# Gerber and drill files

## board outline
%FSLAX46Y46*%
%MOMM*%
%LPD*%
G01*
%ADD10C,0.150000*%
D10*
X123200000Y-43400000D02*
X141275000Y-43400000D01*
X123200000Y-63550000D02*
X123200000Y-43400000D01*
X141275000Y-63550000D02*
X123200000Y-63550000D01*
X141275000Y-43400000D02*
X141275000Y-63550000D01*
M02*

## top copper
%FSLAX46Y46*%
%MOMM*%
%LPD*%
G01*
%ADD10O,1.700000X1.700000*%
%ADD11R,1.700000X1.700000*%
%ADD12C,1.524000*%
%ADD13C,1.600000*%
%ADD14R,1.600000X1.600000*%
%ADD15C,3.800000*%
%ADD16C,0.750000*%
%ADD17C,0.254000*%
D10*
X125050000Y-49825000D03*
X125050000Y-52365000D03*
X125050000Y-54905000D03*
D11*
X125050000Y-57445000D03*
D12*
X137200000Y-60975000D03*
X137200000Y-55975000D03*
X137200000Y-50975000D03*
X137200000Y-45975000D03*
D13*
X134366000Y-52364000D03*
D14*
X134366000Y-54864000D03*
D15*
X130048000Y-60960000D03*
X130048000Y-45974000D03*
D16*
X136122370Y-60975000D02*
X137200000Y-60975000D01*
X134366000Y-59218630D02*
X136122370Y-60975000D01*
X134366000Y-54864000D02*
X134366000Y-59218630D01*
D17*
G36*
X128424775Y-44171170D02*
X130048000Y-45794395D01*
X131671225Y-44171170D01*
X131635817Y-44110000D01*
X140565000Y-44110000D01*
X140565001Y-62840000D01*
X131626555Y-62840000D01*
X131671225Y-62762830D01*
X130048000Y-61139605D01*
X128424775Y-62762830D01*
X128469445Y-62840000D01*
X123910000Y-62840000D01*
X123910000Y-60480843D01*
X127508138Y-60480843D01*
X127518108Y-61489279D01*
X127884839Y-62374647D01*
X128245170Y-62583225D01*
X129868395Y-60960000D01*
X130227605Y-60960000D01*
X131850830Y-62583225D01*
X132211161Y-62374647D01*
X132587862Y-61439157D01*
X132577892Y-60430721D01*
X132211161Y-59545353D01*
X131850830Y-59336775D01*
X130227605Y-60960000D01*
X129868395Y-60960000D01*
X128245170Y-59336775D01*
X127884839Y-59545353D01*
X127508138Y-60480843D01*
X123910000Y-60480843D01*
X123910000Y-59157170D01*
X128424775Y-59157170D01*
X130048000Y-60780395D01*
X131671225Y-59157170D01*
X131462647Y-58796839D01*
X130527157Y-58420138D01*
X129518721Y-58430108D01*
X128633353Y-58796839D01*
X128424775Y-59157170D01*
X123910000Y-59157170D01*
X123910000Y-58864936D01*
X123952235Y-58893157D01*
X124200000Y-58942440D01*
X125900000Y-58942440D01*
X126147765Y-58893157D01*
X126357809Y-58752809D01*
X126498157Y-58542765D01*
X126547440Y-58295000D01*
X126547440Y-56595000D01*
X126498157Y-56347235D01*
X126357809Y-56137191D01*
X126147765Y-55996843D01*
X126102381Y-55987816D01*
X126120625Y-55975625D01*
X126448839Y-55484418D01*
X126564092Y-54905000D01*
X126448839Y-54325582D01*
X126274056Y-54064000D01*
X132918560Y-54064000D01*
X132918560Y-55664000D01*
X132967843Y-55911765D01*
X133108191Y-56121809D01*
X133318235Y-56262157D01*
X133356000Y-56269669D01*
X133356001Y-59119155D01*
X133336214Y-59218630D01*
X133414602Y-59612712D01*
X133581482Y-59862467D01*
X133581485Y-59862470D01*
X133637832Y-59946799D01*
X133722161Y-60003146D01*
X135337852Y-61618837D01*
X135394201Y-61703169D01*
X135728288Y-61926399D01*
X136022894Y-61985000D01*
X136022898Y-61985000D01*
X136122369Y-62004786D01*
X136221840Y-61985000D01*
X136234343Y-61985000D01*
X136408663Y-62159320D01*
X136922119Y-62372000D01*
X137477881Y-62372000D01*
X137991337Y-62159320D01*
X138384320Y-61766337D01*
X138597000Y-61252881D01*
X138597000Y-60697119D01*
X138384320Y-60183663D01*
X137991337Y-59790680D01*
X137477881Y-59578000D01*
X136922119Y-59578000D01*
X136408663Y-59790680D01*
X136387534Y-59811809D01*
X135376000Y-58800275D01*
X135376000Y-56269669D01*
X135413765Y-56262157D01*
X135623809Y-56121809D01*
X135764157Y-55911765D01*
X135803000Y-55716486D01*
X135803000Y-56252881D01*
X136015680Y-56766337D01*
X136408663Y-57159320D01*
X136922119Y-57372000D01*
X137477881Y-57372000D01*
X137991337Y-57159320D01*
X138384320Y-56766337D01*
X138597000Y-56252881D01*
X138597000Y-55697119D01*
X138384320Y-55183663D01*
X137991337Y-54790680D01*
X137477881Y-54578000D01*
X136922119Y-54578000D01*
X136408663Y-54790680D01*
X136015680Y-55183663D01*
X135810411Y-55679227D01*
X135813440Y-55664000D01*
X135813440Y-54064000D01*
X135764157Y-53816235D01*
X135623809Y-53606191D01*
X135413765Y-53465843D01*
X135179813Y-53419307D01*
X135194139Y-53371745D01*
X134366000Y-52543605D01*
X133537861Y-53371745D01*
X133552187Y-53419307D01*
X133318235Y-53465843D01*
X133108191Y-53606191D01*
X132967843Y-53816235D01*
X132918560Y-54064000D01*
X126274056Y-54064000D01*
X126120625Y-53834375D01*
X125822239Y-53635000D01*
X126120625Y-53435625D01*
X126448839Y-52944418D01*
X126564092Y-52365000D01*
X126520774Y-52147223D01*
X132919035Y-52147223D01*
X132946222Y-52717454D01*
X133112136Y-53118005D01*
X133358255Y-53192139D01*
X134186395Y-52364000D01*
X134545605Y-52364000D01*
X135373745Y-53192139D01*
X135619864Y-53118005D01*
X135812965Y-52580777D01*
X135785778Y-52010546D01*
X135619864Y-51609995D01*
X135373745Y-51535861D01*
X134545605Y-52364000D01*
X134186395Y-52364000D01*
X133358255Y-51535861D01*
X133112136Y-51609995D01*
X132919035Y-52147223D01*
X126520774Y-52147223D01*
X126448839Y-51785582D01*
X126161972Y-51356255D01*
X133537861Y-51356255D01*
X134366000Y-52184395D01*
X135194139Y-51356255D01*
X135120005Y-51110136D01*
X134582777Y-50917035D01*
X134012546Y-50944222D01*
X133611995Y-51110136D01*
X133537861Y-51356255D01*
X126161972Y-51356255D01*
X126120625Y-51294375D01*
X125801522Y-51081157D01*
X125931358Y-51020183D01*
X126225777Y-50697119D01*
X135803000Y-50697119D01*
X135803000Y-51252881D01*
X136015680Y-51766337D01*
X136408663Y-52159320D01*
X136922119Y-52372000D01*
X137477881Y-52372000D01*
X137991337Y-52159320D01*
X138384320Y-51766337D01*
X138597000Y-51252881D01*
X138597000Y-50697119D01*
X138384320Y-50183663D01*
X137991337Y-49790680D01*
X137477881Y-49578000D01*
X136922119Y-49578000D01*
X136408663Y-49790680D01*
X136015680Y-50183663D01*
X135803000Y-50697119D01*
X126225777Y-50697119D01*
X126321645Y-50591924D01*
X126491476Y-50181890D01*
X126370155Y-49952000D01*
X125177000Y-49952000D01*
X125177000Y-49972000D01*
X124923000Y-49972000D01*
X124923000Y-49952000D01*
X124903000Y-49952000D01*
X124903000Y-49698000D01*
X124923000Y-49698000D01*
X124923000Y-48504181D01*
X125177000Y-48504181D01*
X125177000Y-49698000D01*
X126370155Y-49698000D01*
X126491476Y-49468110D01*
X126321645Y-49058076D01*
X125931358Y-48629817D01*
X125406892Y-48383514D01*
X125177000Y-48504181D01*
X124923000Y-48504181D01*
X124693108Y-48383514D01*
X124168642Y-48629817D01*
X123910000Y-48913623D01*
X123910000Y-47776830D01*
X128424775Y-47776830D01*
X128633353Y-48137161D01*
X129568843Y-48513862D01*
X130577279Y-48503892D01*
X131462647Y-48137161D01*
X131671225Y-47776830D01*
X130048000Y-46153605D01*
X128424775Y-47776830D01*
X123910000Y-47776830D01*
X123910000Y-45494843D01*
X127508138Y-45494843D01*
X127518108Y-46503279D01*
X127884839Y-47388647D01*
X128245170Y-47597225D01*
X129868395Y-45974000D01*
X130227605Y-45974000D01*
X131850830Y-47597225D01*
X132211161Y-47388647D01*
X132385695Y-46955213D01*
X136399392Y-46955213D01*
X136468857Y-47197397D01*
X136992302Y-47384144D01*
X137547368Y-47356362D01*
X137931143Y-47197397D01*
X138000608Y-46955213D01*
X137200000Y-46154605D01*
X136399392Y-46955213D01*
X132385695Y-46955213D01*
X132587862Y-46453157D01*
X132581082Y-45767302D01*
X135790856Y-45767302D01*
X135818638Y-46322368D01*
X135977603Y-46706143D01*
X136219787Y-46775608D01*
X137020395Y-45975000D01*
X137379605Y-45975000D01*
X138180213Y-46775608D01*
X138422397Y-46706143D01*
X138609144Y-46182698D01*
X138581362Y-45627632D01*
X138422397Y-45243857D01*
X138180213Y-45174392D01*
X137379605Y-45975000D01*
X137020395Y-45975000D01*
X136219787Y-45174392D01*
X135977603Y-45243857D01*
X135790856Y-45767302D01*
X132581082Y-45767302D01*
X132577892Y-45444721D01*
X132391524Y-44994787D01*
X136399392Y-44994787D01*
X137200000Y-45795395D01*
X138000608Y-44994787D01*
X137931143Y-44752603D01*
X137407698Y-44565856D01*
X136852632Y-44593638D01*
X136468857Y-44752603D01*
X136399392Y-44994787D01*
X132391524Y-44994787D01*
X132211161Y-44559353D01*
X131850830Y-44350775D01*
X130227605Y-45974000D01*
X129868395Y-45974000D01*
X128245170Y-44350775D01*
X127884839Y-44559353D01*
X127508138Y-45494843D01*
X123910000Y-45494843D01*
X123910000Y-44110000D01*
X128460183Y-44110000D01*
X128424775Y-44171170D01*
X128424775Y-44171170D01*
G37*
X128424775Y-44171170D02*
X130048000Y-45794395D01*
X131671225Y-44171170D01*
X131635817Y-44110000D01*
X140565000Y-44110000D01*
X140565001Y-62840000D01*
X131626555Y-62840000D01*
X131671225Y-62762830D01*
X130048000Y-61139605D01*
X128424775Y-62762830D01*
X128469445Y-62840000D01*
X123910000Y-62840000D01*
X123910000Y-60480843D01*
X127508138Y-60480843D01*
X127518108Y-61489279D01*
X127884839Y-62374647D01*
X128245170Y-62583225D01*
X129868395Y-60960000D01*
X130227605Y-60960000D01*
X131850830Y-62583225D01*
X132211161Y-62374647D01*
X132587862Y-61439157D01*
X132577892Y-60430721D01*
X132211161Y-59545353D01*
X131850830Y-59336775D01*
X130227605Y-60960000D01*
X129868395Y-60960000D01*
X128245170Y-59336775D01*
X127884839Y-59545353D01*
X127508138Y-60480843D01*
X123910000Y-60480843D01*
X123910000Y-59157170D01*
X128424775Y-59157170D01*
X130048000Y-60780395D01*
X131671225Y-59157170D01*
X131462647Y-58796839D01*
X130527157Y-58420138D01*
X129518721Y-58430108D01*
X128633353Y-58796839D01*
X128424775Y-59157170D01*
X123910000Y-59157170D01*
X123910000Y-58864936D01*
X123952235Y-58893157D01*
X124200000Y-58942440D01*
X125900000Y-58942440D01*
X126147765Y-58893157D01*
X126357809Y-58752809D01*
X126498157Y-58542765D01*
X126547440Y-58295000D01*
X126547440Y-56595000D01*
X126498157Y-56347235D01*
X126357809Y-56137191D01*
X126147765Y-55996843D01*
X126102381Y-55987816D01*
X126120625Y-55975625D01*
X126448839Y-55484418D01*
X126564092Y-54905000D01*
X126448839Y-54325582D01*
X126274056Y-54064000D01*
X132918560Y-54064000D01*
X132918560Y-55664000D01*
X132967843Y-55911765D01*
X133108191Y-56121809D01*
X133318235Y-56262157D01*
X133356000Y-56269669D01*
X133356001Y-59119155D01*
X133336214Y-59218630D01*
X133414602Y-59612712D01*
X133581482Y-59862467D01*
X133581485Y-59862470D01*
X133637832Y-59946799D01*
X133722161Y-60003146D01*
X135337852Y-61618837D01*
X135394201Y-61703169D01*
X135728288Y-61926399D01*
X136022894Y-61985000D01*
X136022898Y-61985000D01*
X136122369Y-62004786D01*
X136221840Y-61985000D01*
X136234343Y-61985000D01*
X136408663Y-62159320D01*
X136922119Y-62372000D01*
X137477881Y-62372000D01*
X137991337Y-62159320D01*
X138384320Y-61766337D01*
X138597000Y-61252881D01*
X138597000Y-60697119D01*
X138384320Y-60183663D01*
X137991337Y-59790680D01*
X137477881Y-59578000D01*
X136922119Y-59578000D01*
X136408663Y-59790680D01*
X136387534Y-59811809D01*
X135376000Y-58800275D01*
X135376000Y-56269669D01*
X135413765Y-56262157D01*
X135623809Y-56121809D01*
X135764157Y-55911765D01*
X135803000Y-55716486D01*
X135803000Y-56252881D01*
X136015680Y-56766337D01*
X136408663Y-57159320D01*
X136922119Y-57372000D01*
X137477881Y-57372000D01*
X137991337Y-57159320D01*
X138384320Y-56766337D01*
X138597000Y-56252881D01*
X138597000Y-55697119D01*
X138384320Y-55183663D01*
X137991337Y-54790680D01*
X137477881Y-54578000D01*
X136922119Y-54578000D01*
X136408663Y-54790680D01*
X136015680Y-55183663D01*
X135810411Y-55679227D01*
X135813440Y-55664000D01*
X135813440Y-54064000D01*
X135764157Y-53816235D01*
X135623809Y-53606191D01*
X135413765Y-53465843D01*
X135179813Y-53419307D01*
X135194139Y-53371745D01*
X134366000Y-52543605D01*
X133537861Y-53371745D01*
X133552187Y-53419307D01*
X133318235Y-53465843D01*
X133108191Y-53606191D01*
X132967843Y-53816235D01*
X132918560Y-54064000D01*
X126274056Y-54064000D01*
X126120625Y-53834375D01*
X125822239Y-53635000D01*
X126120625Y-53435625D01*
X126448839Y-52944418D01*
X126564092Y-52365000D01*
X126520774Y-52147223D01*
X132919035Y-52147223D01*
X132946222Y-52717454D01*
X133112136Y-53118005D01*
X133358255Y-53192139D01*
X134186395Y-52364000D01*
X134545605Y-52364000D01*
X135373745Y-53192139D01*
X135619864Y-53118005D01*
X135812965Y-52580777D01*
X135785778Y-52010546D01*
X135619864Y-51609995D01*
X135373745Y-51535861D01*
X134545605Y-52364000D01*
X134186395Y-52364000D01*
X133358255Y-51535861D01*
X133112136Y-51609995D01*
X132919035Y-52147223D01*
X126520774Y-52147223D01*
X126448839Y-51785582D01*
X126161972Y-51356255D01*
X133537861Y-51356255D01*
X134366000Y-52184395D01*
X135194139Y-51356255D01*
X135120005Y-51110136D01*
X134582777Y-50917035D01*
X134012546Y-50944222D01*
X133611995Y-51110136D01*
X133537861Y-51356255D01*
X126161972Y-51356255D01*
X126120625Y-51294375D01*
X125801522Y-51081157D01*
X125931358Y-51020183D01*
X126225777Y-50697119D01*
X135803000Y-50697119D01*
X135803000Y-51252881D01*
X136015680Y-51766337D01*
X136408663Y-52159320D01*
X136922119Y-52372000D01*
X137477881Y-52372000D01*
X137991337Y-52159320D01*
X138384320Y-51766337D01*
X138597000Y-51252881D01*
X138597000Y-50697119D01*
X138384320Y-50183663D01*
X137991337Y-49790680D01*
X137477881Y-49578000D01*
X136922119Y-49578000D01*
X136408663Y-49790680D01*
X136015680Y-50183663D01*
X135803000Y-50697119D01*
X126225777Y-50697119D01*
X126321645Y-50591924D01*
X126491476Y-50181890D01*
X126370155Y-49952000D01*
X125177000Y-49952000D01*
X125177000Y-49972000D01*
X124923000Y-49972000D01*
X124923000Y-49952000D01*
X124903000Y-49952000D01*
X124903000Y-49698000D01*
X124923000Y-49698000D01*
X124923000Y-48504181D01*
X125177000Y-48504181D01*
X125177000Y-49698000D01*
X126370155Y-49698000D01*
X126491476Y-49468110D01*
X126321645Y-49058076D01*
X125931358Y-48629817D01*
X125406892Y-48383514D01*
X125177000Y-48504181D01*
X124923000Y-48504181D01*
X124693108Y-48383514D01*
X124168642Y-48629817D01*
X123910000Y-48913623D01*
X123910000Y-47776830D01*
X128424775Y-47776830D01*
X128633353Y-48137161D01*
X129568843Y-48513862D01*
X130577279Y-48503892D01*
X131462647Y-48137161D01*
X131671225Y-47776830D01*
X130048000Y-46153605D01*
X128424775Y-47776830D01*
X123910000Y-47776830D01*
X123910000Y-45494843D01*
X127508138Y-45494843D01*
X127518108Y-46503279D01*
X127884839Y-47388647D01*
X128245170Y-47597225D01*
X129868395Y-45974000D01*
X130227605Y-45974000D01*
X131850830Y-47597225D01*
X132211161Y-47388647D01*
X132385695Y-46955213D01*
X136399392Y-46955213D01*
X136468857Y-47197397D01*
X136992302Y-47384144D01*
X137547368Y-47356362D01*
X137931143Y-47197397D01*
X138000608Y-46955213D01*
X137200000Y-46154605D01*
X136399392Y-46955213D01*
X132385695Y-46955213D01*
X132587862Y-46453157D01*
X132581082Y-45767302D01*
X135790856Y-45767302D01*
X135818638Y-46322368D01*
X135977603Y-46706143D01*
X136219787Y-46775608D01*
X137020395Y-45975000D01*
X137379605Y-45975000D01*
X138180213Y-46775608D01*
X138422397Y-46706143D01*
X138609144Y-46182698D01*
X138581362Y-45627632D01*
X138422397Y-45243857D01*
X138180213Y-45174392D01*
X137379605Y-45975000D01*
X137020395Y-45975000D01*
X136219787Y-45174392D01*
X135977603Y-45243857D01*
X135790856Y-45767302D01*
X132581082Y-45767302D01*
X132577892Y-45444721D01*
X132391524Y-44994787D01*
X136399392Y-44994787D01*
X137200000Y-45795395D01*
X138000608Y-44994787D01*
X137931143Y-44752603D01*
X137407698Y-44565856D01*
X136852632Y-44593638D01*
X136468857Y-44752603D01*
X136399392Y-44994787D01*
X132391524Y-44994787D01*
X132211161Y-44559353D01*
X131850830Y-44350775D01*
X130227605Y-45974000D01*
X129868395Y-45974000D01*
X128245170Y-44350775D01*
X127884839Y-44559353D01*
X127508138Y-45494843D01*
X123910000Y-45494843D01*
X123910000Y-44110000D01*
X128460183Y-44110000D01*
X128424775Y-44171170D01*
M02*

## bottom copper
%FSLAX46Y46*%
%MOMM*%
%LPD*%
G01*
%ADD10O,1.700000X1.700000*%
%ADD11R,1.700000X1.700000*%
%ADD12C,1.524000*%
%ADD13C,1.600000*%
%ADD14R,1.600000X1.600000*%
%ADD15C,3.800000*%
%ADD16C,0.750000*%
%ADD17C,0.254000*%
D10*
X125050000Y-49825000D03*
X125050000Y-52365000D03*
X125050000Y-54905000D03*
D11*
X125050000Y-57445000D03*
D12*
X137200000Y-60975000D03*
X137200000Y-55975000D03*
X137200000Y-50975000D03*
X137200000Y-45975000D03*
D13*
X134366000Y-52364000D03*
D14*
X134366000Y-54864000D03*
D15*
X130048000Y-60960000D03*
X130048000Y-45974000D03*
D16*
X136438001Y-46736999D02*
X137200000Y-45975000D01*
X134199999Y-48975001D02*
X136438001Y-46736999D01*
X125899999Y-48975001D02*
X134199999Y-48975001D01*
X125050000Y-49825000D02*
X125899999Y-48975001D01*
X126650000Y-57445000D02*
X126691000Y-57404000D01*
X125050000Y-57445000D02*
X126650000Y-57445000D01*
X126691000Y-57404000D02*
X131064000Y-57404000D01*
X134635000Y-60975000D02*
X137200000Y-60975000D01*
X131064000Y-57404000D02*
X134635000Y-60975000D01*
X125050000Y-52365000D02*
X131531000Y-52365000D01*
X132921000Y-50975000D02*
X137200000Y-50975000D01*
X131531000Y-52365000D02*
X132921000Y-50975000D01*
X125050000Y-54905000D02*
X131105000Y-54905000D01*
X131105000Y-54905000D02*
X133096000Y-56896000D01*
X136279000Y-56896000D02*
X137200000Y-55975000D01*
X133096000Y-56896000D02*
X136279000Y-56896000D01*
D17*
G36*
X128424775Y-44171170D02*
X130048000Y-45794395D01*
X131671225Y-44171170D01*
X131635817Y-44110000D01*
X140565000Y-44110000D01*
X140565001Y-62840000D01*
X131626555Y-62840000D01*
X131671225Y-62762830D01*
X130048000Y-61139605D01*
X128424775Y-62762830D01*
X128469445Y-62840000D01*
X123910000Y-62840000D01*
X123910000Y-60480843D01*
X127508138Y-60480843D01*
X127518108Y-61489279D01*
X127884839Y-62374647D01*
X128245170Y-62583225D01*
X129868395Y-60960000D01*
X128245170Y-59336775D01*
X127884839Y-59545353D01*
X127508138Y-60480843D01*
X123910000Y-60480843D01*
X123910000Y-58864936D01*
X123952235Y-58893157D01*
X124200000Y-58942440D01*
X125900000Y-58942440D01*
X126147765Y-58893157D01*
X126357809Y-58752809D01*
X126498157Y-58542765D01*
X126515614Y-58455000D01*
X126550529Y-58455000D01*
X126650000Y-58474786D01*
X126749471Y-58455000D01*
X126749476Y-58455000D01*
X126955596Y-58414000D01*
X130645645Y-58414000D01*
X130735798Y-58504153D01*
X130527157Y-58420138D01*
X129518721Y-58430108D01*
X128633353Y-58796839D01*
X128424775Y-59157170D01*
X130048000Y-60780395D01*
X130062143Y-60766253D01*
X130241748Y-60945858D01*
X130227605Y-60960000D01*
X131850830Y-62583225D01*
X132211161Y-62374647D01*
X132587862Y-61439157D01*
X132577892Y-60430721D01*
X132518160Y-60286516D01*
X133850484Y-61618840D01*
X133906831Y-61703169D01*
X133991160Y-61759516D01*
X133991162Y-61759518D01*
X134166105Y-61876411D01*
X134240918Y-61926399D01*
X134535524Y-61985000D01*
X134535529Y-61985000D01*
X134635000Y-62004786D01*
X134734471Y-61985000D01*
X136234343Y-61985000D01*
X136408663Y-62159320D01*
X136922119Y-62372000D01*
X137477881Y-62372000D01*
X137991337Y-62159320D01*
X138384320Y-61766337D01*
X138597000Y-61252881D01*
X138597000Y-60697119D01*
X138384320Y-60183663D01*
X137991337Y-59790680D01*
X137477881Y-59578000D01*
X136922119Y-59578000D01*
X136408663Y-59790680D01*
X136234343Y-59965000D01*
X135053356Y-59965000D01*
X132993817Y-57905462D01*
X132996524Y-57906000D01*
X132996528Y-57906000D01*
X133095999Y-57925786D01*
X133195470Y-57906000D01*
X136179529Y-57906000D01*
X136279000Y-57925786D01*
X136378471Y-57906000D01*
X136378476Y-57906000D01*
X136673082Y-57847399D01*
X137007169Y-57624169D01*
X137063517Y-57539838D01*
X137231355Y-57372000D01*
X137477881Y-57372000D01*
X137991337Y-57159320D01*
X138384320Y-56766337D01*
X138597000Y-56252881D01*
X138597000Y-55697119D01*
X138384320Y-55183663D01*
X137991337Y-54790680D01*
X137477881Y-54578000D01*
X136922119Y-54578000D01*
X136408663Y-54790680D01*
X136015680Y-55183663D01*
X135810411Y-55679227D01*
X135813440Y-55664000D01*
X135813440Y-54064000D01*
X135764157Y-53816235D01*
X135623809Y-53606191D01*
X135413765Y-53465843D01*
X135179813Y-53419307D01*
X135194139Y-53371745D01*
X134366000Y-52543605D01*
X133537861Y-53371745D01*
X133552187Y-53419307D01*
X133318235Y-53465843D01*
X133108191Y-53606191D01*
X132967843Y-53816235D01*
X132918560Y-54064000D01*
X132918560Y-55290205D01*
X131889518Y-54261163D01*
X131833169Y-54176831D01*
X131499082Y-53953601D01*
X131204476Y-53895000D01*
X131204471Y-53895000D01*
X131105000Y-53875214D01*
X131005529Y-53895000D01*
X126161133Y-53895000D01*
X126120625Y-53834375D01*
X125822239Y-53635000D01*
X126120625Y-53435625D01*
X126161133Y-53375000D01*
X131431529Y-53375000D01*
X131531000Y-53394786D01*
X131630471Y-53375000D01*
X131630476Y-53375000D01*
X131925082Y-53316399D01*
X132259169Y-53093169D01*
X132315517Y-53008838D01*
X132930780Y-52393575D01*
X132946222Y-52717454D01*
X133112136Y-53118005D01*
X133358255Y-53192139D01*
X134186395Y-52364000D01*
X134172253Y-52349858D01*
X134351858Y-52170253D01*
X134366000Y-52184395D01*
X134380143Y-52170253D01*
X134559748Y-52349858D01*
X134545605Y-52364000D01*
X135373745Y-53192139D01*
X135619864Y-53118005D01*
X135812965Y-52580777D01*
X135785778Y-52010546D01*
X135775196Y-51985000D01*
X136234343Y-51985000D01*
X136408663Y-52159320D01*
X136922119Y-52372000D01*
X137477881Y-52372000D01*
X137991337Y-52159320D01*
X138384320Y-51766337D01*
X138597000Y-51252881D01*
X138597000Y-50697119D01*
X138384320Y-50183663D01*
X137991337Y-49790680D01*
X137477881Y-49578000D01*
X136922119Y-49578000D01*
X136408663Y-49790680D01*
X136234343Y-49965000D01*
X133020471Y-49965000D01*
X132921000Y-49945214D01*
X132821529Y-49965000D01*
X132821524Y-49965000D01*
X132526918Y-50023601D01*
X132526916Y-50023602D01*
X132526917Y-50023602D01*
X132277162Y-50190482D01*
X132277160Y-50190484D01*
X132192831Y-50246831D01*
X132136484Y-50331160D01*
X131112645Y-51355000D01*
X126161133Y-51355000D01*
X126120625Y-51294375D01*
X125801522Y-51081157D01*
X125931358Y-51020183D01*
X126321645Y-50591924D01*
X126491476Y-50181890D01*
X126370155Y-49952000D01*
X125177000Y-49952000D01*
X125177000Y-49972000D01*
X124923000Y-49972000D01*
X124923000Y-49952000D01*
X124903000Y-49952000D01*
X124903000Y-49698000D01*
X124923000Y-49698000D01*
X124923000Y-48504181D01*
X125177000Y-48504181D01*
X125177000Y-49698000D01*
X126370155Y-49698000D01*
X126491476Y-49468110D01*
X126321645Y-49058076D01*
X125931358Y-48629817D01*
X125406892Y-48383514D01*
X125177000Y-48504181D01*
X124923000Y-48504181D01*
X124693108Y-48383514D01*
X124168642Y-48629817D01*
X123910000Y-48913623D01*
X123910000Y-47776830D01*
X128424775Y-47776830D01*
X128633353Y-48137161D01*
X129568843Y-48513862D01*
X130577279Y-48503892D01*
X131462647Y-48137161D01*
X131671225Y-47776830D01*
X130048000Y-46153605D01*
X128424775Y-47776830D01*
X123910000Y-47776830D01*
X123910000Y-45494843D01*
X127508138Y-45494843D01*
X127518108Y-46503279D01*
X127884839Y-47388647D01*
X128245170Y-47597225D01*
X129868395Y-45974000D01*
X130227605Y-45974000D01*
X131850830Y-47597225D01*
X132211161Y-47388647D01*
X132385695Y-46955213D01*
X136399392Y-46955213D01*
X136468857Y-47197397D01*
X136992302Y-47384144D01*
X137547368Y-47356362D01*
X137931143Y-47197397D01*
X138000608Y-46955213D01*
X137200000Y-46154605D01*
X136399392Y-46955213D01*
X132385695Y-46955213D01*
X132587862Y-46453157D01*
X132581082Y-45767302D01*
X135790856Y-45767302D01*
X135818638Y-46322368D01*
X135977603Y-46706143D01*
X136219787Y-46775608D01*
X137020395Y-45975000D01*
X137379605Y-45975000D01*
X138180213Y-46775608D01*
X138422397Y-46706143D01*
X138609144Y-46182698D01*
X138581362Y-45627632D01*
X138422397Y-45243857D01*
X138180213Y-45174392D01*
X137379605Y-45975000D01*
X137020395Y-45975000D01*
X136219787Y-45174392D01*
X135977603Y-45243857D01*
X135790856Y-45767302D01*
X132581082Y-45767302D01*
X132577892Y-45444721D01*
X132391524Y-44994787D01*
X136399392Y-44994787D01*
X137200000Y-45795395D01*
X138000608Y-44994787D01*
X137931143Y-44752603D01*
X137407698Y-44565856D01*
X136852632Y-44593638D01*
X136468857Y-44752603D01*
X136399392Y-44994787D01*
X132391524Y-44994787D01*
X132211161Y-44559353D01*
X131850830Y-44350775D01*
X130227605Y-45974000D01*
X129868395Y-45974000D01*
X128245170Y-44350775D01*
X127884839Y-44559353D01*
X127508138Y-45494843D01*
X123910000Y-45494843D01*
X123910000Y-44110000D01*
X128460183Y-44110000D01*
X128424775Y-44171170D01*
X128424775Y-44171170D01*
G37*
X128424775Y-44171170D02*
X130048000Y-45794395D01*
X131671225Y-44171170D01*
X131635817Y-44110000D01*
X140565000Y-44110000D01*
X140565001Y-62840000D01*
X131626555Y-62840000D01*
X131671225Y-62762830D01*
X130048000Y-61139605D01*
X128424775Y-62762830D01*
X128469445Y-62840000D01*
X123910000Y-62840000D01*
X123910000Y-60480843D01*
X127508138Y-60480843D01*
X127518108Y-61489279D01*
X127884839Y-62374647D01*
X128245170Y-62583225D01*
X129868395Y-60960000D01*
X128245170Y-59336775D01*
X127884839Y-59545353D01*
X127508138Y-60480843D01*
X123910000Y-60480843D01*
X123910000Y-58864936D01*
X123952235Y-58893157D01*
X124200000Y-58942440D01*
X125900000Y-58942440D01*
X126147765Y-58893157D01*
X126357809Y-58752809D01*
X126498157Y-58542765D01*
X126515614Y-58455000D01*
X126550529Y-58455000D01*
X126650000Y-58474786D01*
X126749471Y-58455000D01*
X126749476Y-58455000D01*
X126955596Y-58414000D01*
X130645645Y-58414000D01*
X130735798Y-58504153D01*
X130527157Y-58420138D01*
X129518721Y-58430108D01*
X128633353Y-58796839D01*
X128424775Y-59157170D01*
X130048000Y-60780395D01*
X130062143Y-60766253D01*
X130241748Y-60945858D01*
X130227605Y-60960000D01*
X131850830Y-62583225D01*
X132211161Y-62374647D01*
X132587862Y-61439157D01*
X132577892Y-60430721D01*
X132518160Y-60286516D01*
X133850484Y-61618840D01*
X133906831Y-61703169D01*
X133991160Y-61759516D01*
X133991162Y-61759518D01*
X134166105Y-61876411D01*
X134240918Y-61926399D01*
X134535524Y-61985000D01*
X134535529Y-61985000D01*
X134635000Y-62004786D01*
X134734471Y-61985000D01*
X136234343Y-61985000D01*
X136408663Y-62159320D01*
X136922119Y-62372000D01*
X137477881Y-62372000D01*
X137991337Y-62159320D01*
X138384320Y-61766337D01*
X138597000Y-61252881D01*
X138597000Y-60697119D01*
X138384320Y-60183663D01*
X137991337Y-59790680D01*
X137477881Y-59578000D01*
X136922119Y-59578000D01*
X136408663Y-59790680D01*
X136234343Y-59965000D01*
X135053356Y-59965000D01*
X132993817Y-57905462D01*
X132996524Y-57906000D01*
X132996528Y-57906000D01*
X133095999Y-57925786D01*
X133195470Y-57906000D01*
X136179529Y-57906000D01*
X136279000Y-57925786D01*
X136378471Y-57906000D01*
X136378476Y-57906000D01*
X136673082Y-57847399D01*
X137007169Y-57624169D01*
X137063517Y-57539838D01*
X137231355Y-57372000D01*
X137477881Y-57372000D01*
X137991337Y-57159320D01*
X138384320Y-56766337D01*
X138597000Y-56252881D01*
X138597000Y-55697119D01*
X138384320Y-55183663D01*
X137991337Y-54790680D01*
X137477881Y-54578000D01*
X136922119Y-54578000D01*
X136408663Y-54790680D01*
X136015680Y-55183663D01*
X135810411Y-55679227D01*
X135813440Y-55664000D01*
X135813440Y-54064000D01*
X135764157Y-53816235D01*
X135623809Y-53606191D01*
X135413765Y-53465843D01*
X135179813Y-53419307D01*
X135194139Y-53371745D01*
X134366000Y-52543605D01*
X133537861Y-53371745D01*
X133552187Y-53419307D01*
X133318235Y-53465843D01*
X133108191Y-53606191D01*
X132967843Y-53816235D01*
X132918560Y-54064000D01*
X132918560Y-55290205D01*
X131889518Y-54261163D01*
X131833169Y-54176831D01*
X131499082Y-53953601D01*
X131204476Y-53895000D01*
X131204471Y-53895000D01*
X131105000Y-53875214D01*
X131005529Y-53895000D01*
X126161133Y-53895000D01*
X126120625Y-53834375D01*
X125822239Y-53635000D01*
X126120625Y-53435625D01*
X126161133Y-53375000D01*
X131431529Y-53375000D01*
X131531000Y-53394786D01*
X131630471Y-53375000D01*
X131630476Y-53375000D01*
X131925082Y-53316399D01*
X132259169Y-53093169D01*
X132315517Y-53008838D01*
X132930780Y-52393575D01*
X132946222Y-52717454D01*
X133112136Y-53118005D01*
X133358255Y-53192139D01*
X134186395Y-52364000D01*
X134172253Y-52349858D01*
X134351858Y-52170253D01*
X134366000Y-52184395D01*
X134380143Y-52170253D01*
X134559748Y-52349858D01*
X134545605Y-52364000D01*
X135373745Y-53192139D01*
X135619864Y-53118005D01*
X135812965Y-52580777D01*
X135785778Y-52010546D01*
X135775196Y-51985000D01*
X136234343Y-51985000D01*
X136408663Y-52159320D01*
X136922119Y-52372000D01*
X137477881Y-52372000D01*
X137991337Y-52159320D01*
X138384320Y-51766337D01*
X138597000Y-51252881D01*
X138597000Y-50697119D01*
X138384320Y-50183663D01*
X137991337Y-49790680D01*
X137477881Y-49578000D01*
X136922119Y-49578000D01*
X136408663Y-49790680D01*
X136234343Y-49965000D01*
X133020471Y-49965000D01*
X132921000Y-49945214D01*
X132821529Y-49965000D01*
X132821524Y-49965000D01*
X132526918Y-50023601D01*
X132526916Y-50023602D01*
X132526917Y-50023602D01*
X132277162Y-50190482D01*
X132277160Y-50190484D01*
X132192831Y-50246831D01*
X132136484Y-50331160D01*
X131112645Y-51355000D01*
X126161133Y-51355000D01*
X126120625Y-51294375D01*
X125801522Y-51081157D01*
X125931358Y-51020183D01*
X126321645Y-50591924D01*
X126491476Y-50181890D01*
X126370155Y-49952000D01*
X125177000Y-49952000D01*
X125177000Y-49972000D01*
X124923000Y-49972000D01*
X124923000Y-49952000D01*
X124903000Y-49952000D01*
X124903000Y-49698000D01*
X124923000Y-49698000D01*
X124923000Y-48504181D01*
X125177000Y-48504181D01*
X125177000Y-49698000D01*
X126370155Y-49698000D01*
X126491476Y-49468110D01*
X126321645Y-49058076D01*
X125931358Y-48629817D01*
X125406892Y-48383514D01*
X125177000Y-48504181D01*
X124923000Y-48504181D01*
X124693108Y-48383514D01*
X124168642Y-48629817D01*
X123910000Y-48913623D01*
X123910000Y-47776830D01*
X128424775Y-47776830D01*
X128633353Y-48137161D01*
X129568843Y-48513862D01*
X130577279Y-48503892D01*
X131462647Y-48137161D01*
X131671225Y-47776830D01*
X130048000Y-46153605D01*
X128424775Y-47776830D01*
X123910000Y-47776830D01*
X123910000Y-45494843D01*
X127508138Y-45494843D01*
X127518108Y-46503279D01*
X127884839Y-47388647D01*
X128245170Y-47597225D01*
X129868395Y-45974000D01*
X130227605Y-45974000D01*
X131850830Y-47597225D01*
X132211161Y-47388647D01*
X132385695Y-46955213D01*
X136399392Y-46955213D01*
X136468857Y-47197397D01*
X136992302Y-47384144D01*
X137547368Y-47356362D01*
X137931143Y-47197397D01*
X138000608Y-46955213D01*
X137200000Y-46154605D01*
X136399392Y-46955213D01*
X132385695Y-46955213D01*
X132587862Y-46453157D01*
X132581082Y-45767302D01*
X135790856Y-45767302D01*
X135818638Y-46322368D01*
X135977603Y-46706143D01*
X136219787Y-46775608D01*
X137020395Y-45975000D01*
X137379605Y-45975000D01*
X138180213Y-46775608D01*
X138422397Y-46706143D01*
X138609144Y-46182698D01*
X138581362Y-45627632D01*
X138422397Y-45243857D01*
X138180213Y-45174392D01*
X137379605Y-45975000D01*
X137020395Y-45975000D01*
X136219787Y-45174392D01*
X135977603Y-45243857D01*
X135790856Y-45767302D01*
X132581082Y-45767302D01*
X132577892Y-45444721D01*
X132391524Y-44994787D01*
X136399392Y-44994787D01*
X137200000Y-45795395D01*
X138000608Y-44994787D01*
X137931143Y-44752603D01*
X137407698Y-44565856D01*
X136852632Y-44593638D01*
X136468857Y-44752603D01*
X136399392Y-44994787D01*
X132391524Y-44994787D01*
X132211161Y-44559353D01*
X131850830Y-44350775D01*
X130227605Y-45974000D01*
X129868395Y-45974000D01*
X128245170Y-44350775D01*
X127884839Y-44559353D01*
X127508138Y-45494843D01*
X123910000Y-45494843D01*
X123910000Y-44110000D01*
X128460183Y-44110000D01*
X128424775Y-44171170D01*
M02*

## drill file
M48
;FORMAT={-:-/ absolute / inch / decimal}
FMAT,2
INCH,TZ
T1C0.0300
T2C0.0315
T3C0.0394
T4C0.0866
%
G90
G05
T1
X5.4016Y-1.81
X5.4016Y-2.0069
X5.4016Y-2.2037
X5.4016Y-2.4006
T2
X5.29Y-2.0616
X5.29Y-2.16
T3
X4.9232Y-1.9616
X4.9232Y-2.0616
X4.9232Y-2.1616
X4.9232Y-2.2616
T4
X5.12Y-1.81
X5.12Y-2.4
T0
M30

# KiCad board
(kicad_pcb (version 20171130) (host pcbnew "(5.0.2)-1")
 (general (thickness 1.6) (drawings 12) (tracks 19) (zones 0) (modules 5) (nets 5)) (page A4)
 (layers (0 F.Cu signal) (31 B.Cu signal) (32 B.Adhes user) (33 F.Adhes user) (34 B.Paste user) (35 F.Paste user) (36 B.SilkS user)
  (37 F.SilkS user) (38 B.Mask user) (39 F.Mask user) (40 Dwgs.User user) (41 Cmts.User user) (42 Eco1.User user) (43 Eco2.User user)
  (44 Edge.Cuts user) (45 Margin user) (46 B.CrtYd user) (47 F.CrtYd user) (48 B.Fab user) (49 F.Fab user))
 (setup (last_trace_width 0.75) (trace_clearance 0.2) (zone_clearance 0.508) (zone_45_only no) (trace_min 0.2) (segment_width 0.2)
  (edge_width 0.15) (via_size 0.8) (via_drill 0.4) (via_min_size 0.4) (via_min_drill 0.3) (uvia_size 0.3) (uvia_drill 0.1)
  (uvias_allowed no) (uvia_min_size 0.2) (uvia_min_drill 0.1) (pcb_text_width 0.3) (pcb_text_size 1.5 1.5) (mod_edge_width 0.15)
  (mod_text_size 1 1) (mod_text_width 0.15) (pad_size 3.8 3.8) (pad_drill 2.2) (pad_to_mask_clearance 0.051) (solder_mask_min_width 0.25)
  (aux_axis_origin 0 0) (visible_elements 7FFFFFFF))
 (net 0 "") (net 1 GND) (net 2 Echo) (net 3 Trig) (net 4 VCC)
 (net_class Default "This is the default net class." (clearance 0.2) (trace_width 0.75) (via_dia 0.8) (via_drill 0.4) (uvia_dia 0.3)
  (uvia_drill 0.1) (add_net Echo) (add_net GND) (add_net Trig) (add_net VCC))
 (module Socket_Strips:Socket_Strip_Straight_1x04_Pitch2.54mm (layer B.Cu) (at 125.05 57.445)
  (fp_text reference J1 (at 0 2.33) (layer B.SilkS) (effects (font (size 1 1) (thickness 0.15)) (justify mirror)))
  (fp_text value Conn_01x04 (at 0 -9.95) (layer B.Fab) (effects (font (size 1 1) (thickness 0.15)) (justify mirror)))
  (pad 4 thru_hole oval (at 0 -7.62) (size 1.7 1.7) (drill 1) (layers *.Cu *.Mask) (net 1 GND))
  (pad 3 thru_hole oval (at 0 -5.08) (size 1.7 1.7) (drill 1) (layers *.Cu *.Mask) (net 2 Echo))
  (pad 2 thru_hole oval (at 0 -2.54) (size 1.7 1.7) (drill 1) (layers *.Cu *.Mask) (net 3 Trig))
  (pad 1 thru_hole rect (at 0 0) (size 1.7 1.7) (drill 1) (layers *.Cu *.Mask) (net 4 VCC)))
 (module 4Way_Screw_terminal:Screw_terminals (layer B.Cu) (at 137.2 53.475)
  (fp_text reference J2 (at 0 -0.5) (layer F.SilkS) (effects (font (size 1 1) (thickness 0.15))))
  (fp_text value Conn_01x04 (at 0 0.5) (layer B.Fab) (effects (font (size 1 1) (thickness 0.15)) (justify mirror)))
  (pad 1 thru_hole circle (at 0 7.5) (size 1.524 1.524) (drill 0.762) (layers *.Cu *.Mask) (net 4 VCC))
  (pad 2 thru_hole circle (at 0 2.5) (size 1.524 1.524) (drill 0.762) (layers *.Cu *.Mask) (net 3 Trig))
  (pad 3 thru_hole circle (at 0 -2.5) (size 1.524 1.524) (drill 0.762) (layers *.Cu *.Mask) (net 2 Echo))
  (pad 4 thru_hole circle (at 0 -7.5) (size 1.524 1.524) (drill 0.762) (layers *.Cu *.Mask) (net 1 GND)))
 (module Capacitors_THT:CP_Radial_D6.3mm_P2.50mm (layer F.Cu) (at 134.366 54.864 90)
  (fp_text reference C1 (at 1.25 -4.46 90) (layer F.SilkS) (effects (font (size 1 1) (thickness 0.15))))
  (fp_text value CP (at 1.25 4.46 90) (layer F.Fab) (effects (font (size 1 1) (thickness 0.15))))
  (pad 2 thru_hole circle (at 2.5 0 90) (size 1.6 1.6) (drill 0.8) (layers *.Cu *.Mask) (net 1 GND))
  (pad 1 thru_hole rect (at 0 0 90) (size 1.6 1.6) (drill 0.8) (layers *.Cu *.Mask) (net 4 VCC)))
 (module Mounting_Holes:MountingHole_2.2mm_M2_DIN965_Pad (layer F.Cu) (at 130.048 60.96)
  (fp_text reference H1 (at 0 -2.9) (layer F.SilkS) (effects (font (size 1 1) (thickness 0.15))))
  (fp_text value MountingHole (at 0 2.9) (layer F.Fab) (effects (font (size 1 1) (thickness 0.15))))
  (pad 1 thru_hole circle (at 0 0) (size 3.8 3.8) (drill 2.2) (layers *.Cu *.Mask) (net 1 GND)))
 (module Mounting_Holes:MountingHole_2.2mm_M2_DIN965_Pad (layer F.Cu) (at 130.048 45.974)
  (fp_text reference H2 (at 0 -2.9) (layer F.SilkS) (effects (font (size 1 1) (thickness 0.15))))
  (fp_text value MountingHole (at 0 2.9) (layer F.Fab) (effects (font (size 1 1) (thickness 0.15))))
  (pad 1 thru_hole circle (at 0 0) (size 3.8 3.8) (drill 2.2) (layers *.Cu *.Mask) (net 1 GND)))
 (gr_line (start 123.2 43.4) (end 141.275 43.4) (layer Edge.Cuts) (width 0.15))
 (gr_line (start 123.2 63.55) (end 123.2 43.4) (layer Edge.Cuts) (width 0.15))
 (gr_line (start 141.275 63.55) (end 123.2 63.55) (layer Edge.Cuts) (width 0.15))
 (gr_line (start 141.275 43.4) (end 141.275 63.55) (layer Edge.Cuts) (width 0.15))
 (segment (start 136.438001 46.736999) (end 137.2 45.975) (width 0.75) (layer B.Cu) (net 1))
 (segment (start 134.199999 48.975001) (end 136.438001 46.736999) (width 0.75) (layer B.Cu) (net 1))
 (segment (start 125.899999 48.975001) (end 134.199999 48.975001) (width 0.75) (layer B.Cu) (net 1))
 (segment (start 125.05 49.825) (end 125.899999 48.975001) (width 0.75) (layer B.Cu) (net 1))
 (segment (start 136.12237 60.975) (end 137.2 60.975) (width 0.75) (layer F.Cu) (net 4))
 (segment (start 134.366 59.21863) (end 136.12237 60.975) (width 0.75) (layer F.Cu) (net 4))
 (segment (start 134.366 54.864) (end 134.366 59.21863) (width 0.75) (layer F.Cu) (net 4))
 (segment (start 126.65 57.445) (end 126.691 57.404) (width 0.75) (layer B.Cu) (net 4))
 (segment (start 125.05 57.445) (end 126.65 57.445) (width 0.75) (layer B.Cu) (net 4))
 (segment (start 126.691 57.404) (end 131.064 57.404) (width 0.75) (layer B.Cu) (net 4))
 (segment (start 134.635 60.975) (end 137.2 60.975) (width 0.75) (layer B.Cu) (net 4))
 (segment (start 131.064 57.404) (end 134.635 60.975) (width 0.75) (layer B.Cu) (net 4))
 (segment (start 125.05 52.365) (end 131.531 52.365) (width 0.75) (layer B.Cu) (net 2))
 (segment (start 132.921 50.975) (end 137.2 50.975) (width 0.75) (layer B.Cu) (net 2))
 (segment (start 131.531 52.365) (end 132.921 50.975) (width 0.75) (layer B.Cu) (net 2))
 (segment (start 125.05 54.905) (end 131.105 54.905) (width 0.75) (layer B.Cu) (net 3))
 (segment (start 131.105 54.905) (end 133.096 56.896) (width 0.75) (layer B.Cu) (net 3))
 (segment (start 136.279 56.896) (end 137.2 55.975) (width 0.75) (layer B.Cu) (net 3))
 (segment (start 133.096 56.896) (end 136.279 56.896) (width 0.75) (layer B.Cu) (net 3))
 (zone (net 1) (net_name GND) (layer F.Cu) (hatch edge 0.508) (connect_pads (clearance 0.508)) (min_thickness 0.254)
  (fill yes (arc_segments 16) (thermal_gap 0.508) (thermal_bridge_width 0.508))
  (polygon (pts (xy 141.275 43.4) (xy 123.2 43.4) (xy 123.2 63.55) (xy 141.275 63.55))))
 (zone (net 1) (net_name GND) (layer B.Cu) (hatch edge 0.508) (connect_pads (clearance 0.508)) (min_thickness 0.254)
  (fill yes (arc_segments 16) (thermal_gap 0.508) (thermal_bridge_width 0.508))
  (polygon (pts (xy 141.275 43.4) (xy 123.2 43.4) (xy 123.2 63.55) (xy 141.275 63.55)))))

